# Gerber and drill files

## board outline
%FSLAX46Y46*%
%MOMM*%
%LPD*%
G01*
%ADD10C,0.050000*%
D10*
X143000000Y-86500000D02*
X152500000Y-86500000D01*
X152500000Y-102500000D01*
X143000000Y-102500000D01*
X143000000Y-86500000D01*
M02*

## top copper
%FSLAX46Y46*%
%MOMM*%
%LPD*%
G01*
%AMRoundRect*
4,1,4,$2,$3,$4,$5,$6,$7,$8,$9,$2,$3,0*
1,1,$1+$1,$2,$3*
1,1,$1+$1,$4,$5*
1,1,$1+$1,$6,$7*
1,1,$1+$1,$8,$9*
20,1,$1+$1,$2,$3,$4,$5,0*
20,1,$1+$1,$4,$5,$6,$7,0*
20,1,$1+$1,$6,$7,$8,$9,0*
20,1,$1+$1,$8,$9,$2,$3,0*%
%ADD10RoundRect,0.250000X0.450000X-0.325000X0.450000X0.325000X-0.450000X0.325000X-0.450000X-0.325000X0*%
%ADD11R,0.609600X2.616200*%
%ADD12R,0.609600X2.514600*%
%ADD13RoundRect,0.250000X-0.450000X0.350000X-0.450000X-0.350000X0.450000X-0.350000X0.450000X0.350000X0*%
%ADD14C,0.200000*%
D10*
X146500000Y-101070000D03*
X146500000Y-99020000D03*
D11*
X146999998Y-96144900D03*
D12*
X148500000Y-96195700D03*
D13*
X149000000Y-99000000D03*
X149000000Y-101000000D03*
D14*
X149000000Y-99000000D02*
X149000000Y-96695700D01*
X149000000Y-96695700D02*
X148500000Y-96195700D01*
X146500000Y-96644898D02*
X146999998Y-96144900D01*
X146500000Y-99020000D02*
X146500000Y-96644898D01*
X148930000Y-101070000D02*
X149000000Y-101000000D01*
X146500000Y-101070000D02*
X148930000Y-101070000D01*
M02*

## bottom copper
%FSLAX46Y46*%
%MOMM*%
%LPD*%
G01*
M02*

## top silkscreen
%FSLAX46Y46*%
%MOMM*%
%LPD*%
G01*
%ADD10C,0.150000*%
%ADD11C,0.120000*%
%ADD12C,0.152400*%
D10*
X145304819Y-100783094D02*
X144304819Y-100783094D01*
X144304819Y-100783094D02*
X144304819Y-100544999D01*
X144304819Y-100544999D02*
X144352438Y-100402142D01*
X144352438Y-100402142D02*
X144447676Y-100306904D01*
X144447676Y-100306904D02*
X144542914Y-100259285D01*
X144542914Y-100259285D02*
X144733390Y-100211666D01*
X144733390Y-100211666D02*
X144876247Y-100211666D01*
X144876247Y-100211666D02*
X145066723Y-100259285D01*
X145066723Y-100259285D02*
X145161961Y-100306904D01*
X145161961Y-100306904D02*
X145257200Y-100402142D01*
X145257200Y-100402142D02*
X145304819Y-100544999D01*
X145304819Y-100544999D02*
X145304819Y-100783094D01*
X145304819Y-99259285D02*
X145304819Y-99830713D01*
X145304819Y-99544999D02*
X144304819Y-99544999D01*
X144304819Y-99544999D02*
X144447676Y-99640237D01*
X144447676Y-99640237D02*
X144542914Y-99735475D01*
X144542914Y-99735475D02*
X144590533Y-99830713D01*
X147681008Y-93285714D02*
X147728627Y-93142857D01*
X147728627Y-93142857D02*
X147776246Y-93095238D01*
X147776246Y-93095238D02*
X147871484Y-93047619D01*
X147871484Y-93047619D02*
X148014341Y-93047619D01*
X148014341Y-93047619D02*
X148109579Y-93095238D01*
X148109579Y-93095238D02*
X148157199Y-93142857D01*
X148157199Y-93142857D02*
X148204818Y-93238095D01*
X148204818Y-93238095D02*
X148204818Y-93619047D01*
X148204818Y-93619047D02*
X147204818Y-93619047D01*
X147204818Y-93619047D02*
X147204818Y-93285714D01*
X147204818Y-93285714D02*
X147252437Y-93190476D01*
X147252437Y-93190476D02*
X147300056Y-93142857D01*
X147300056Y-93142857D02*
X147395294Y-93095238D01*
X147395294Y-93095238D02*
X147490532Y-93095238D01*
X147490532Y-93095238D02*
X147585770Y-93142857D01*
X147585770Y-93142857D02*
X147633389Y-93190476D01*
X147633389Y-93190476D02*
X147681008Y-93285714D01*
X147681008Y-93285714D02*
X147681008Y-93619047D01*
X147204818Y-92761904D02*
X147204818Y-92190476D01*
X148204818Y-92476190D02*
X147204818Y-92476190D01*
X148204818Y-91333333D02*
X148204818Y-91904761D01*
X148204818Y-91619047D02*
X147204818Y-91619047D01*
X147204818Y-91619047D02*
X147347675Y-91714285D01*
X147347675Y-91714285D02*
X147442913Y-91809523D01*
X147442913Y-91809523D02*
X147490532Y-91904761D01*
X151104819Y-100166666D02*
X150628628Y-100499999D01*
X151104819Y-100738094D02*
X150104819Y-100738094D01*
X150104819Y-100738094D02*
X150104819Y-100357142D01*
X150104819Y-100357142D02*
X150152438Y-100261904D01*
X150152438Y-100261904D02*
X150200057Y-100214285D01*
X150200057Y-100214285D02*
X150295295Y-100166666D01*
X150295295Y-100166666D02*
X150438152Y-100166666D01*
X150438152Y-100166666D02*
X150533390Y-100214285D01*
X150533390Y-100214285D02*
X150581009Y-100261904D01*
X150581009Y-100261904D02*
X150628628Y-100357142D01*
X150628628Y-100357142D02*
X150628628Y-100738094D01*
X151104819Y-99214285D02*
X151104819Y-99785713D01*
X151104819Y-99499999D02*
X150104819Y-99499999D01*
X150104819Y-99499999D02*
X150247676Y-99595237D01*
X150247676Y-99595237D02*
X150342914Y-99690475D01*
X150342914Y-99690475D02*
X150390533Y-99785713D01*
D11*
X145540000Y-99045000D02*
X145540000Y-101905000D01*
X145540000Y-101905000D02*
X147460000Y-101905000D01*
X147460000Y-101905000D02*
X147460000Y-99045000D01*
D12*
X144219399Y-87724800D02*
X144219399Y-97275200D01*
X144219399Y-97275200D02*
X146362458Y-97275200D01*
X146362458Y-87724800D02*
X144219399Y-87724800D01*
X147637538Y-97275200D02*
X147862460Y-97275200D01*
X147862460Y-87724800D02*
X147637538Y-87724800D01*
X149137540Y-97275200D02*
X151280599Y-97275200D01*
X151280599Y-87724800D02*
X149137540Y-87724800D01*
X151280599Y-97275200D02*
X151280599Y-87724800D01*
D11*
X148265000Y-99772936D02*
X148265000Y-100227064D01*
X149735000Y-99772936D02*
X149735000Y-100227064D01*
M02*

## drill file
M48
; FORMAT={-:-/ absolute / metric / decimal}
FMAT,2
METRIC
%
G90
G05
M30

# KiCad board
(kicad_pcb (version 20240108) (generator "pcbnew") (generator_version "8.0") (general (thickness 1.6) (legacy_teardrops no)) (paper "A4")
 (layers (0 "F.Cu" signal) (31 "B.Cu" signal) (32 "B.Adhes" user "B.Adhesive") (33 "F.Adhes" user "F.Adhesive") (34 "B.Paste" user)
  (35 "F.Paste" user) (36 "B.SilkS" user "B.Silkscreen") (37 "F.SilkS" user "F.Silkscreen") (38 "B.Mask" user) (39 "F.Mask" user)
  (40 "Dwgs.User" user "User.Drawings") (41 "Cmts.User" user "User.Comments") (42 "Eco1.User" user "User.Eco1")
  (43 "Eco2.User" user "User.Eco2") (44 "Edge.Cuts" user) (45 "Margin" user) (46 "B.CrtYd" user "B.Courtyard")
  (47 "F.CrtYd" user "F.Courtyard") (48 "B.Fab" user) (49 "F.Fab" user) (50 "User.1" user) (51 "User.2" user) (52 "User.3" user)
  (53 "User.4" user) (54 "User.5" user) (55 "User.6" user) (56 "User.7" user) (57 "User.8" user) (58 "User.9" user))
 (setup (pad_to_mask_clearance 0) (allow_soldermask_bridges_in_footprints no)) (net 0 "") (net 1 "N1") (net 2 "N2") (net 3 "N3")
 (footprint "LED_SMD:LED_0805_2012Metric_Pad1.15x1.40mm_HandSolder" (layer "F.Cu") (at 146.5 100.045 90)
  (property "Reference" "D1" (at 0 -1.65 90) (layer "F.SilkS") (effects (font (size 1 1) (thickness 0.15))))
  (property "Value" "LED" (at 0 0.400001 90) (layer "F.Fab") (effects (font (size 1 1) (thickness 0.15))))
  (fp_line (start 1 -0.96) (end -1.86 -0.96) (stroke (width 0.12) (type solid)) (layer "F.SilkS"))
  (fp_line (start -1.86 -0.96) (end -1.86 0.96) (stroke (width 0.12) (type solid)) (layer "F.SilkS"))
  (fp_line (start -1.86 0.96) (end 1 0.96) (stroke (width 0.12) (type solid)) (layer "F.SilkS"))
  (pad "1" smd roundrect (at -1.025 0 90) (size 1.15 1.4) (layers "F.Cu" "F.Paste" "F.Mask") (roundrect_rratio 0.217391) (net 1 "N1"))
  (pad "2" smd roundrect (at 1.025 0 90) (size 1.15 1.4) (layers "F.Cu" "F.Paste" "F.Mask") (roundrect_rratio 0.217391) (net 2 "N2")))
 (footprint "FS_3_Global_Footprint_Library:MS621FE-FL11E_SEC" (layer "F.Cu") (at 147.749999 92.5 90)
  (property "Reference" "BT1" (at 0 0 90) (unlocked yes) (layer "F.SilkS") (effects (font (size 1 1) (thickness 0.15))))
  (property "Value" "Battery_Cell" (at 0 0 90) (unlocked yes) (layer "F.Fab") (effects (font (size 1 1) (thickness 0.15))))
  (fp_line (start 4.7752 -3.5306) (end -4.7752 -3.5306) (stroke (width 0.1524) (type solid)) (layer "F.SilkS"))
  (fp_line (start -4.7752 -3.5306) (end -4.7752 -1.387541) (stroke (width 0.1524) (type solid)) (layer "F.SilkS"))
  (fp_line (start 4.7752 -1.387541) (end 4.7752 -3.5306) (stroke (width 0.1524) (type solid)) (layer "F.SilkS"))
  (fp_line (start -4.7752 -0.112461) (end -4.7752 0.112461) (stroke (width 0.1524) (type solid)) (layer "F.SilkS"))
  (fp_line (start 4.7752 0.112461) (end 4.7752 -0.112461) (stroke (width 0.1524) (type solid)) (layer "F.SilkS"))
  (fp_line (start -4.7752 1.387541) (end -4.7752 3.5306) (stroke (width 0.1524) (type solid)) (layer "F.SilkS"))
  (fp_line (start 4.7752 3.5306) (end 4.7752 1.387541) (stroke (width 0.1524) (type solid)) (layer "F.SilkS"))
  (fp_line (start -4.7752 3.5306) (end 4.7752 3.5306) (stroke (width 0.1524) (type solid)) (layer "F.SilkS"))
  (pad "1" smd rect (at -3.6449 -0.750001 90) (size 2.6162 0.6096) (layers "F.Cu" "F.Paste" "F.Mask") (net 2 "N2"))
  (pad "2" smd rect (at -3.6957 0.750001 90) (size 2.5146 0.6096) (layers "F.Cu" "F.Paste" "F.Mask") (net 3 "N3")))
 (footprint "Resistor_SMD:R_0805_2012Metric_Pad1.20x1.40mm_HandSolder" (layer "F.Cu") (at 149 100 -90)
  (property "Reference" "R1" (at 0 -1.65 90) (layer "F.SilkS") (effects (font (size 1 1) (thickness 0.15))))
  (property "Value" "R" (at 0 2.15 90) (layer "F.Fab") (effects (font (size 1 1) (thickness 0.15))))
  (fp_line (start -0.227064 0.735) (end 0.227064 0.735) (stroke (width 0.12) (type solid)) (layer "F.SilkS"))
  (fp_line (start -0.227064 -0.735) (end 0.227064 -0.735) (stroke (width 0.12) (type solid)) (layer "F.SilkS"))
  (pad "1" smd roundrect (at -1 0 270) (size 1.2 1.4) (layers "F.Cu" "F.Paste" "F.Mask") (roundrect_rratio 0.208333) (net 3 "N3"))
  (pad "2" smd roundrect (at 1 0 270) (size 1.2 1.4) (layers "F.Cu" "F.Paste" "F.Mask") (roundrect_rratio 0.208333) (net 1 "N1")))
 (gr_rect (start 143 86.5) (end 152.5 102.5) (stroke (width 0.05) (type default)) (fill none) (layer "Edge.Cuts"))
 (segment (start 149 99) (end 149 96.6957) (width 0.2) (layer "F.Cu") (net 3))
 (segment (start 149 96.6957) (end 148.5 96.1957) (width 0.2) (layer "F.Cu") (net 3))
 (segment (start 146.5 96.644898) (end 146.999998 96.1449) (width 0.2) (layer "F.Cu") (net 2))
 (segment (start 146.5 99.02) (end 146.5 96.644898) (width 0.2) (layer "F.Cu") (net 2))
 (segment (start 148.93 101.07) (end 149 101) (width 0.2) (layer "F.Cu") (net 1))
 (segment (start 146.5 101.07) (end 148.93 101.07) (width 0.2) (layer "F.Cu") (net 1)))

